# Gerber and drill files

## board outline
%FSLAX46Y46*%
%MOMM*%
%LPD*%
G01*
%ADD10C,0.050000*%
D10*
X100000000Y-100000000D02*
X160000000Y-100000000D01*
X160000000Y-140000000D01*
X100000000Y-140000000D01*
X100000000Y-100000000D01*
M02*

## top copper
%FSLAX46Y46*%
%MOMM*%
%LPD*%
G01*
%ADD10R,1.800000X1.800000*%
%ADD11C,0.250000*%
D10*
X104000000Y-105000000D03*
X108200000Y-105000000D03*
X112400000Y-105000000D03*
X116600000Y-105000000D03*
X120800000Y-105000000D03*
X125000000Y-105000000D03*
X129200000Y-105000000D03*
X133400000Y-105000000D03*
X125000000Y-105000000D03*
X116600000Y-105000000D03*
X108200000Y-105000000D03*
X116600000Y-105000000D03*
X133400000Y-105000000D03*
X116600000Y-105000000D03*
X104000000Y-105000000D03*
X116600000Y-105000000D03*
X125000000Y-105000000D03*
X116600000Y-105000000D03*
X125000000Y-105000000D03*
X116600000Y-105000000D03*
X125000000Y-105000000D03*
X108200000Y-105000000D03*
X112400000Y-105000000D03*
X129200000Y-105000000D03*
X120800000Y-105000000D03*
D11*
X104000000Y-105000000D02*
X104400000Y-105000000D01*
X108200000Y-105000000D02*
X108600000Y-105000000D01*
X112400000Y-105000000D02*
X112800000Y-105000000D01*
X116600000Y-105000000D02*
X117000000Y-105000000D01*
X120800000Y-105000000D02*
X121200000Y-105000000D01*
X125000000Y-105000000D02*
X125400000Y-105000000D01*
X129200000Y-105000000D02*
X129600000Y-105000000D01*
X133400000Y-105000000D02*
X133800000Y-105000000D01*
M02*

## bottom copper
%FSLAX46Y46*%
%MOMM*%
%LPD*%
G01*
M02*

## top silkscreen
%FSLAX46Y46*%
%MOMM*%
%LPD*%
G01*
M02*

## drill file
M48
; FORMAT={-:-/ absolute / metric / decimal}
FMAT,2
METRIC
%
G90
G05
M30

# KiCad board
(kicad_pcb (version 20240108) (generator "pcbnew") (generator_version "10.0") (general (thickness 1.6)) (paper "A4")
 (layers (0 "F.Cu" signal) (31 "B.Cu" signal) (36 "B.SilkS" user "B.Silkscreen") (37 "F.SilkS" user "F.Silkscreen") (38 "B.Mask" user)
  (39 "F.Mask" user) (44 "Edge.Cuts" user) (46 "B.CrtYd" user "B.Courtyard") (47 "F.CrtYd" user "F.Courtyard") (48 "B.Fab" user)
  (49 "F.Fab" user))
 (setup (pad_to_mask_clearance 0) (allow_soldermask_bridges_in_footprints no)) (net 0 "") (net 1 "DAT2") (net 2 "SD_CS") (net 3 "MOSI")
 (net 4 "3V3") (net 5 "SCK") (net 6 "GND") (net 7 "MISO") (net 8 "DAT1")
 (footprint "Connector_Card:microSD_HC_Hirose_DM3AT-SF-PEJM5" (layer "F.Cu") (at 100 100)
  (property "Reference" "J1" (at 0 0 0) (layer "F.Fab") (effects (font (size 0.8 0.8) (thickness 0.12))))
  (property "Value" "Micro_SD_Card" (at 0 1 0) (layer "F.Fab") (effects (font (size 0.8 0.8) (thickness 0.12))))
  (pad "1" smd rect (at 4.000 5.000) (size 1.8 1.8) (layers "F.Cu" "F.Paste" "F.Mask") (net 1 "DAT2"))
  (pad "2" smd rect (at 8.200 5.000) (size 1.8 1.8) (layers "F.Cu" "F.Paste" "F.Mask") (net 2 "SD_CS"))
  (pad "3" smd rect (at 12.400 5.000) (size 1.8 1.8) (layers "F.Cu" "F.Paste" "F.Mask") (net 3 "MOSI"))
  (pad "4" smd rect (at 16.600 5.000) (size 1.8 1.8) (layers "F.Cu" "F.Paste" "F.Mask") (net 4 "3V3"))
  (pad "5" smd rect (at 20.800 5.000) (size 1.8 1.8) (layers "F.Cu" "F.Paste" "F.Mask") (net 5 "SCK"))
  (pad "6" smd rect (at 25.000 5.000) (size 1.8 1.8) (layers "F.Cu" "F.Paste" "F.Mask") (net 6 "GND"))
  (pad "7" smd rect (at 29.200 5.000) (size 1.8 1.8) (layers "F.Cu" "F.Paste" "F.Mask") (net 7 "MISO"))
  (pad "8" smd rect (at 33.400 5.000) (size 1.8 1.8) (layers "F.Cu" "F.Paste" "F.Mask") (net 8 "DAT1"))
  (pad "SH" smd rect (at 25.000 5.000) (size 1.8 1.8) (layers "F.Cu" "F.Paste" "F.Mask") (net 6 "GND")))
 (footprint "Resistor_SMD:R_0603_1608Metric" (layer "F.Cu") (at 100 100)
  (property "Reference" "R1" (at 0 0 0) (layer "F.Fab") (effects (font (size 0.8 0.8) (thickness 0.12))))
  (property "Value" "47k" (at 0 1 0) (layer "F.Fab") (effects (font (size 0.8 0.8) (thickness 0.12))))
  (pad "1" smd rect (at 16.600 5.000) (size 1.8 1.8) (layers "F.Cu" "F.Paste" "F.Mask") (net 4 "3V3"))
  (pad "2" smd rect (at 8.200 5.000) (size 1.8 1.8) (layers "F.Cu" "F.Paste" "F.Mask") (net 2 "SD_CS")))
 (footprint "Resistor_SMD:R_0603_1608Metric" (layer "F.Cu") (at 100 100)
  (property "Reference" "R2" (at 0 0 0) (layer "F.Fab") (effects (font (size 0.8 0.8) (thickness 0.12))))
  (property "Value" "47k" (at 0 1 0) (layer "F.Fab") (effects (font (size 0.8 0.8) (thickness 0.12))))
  (pad "1" smd rect (at 16.600 5.000) (size 1.8 1.8) (layers "F.Cu" "F.Paste" "F.Mask") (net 4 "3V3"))
  (pad "2" smd rect (at 33.400 5.000) (size 1.8 1.8) (layers "F.Cu" "F.Paste" "F.Mask") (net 8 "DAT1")))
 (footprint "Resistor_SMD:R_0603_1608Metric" (layer "F.Cu") (at 100 100)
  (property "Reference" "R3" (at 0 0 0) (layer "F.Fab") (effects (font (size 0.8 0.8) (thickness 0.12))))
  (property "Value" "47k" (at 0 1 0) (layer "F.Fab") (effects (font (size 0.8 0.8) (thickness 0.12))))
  (pad "1" smd rect (at 16.600 5.000) (size 1.8 1.8) (layers "F.Cu" "F.Paste" "F.Mask") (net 4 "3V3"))
  (pad "2" smd rect (at 4.000 5.000) (size 1.8 1.8) (layers "F.Cu" "F.Paste" "F.Mask") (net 1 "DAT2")))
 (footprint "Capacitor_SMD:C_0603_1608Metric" (layer "F.Cu") (at 100 100)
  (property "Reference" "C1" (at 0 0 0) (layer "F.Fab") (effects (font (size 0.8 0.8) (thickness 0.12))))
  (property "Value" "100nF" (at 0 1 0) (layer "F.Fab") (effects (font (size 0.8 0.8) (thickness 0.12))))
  (pad "1" smd rect (at 16.600 5.000) (size 1.8 1.8) (layers "F.Cu" "F.Paste" "F.Mask") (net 4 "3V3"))
  (pad "2" smd rect (at 25.000 5.000) (size 1.8 1.8) (layers "F.Cu" "F.Paste" "F.Mask") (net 6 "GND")))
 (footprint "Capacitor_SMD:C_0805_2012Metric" (layer "F.Cu") (at 100 100)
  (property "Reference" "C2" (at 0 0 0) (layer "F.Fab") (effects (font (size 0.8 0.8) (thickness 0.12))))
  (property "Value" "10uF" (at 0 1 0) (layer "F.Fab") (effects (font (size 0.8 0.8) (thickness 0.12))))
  (pad "1" smd rect (at 16.600 5.000) (size 1.8 1.8) (layers "F.Cu" "F.Paste" "F.Mask") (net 4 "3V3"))
  (pad "2" smd rect (at 25.000 5.000) (size 1.8 1.8) (layers "F.Cu" "F.Paste" "F.Mask") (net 6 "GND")))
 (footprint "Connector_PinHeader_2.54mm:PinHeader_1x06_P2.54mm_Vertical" (layer "F.Cu") (at 100 100)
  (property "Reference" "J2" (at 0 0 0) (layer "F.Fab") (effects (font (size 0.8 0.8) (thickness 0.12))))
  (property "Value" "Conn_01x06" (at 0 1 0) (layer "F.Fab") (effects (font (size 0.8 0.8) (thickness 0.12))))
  (pad "1" smd rect (at 16.600 5.000) (size 1.8 1.8) (layers "F.Cu" "F.Paste" "F.Mask") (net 4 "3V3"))
  (pad "2" smd rect (at 25.000 5.000) (size 1.8 1.8) (layers "F.Cu" "F.Paste" "F.Mask") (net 6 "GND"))
  (pad "3" smd rect (at 8.200 5.000) (size 1.8 1.8) (layers "F.Cu" "F.Paste" "F.Mask") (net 2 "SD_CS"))
  (pad "4" smd rect (at 12.400 5.000) (size 1.8 1.8) (layers "F.Cu" "F.Paste" "F.Mask") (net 3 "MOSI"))
  (pad "5" smd rect (at 29.200 5.000) (size 1.8 1.8) (layers "F.Cu" "F.Paste" "F.Mask") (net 7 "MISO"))
  (pad "6" smd rect (at 20.800 5.000) (size 1.8 1.8) (layers "F.Cu" "F.Paste" "F.Mask") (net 5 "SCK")))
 (gr_rect (start 100 100) (end 160 140) (stroke (width 0.05) (type default)) (fill none) (layer "Edge.Cuts"))
 (segment (start 104.000 105.000) (end 104.400 105.000) (width 0.25) (layer "F.Cu") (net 1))
 (segment (start 108.200 105.000) (end 108.600 105.000) (width 0.25) (layer "F.Cu") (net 2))
 (segment (start 112.400 105.000) (end 112.800 105.000) (width 0.25) (layer "F.Cu") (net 3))
 (segment (start 116.600 105.000) (end 117.000 105.000) (width 0.25) (layer "F.Cu") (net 4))
 (segment (start 120.800 105.000) (end 121.200 105.000) (width 0.25) (layer "F.Cu") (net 5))
 (segment (start 125.000 105.000) (end 125.400 105.000) (width 0.25) (layer "F.Cu") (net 6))
 (segment (start 129.200 105.000) (end 129.600 105.000) (width 0.25) (layer "F.Cu") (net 7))
 (segment (start 133.400 105.000) (end 133.800 105.000) (width 0.25) (layer "F.Cu") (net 8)))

